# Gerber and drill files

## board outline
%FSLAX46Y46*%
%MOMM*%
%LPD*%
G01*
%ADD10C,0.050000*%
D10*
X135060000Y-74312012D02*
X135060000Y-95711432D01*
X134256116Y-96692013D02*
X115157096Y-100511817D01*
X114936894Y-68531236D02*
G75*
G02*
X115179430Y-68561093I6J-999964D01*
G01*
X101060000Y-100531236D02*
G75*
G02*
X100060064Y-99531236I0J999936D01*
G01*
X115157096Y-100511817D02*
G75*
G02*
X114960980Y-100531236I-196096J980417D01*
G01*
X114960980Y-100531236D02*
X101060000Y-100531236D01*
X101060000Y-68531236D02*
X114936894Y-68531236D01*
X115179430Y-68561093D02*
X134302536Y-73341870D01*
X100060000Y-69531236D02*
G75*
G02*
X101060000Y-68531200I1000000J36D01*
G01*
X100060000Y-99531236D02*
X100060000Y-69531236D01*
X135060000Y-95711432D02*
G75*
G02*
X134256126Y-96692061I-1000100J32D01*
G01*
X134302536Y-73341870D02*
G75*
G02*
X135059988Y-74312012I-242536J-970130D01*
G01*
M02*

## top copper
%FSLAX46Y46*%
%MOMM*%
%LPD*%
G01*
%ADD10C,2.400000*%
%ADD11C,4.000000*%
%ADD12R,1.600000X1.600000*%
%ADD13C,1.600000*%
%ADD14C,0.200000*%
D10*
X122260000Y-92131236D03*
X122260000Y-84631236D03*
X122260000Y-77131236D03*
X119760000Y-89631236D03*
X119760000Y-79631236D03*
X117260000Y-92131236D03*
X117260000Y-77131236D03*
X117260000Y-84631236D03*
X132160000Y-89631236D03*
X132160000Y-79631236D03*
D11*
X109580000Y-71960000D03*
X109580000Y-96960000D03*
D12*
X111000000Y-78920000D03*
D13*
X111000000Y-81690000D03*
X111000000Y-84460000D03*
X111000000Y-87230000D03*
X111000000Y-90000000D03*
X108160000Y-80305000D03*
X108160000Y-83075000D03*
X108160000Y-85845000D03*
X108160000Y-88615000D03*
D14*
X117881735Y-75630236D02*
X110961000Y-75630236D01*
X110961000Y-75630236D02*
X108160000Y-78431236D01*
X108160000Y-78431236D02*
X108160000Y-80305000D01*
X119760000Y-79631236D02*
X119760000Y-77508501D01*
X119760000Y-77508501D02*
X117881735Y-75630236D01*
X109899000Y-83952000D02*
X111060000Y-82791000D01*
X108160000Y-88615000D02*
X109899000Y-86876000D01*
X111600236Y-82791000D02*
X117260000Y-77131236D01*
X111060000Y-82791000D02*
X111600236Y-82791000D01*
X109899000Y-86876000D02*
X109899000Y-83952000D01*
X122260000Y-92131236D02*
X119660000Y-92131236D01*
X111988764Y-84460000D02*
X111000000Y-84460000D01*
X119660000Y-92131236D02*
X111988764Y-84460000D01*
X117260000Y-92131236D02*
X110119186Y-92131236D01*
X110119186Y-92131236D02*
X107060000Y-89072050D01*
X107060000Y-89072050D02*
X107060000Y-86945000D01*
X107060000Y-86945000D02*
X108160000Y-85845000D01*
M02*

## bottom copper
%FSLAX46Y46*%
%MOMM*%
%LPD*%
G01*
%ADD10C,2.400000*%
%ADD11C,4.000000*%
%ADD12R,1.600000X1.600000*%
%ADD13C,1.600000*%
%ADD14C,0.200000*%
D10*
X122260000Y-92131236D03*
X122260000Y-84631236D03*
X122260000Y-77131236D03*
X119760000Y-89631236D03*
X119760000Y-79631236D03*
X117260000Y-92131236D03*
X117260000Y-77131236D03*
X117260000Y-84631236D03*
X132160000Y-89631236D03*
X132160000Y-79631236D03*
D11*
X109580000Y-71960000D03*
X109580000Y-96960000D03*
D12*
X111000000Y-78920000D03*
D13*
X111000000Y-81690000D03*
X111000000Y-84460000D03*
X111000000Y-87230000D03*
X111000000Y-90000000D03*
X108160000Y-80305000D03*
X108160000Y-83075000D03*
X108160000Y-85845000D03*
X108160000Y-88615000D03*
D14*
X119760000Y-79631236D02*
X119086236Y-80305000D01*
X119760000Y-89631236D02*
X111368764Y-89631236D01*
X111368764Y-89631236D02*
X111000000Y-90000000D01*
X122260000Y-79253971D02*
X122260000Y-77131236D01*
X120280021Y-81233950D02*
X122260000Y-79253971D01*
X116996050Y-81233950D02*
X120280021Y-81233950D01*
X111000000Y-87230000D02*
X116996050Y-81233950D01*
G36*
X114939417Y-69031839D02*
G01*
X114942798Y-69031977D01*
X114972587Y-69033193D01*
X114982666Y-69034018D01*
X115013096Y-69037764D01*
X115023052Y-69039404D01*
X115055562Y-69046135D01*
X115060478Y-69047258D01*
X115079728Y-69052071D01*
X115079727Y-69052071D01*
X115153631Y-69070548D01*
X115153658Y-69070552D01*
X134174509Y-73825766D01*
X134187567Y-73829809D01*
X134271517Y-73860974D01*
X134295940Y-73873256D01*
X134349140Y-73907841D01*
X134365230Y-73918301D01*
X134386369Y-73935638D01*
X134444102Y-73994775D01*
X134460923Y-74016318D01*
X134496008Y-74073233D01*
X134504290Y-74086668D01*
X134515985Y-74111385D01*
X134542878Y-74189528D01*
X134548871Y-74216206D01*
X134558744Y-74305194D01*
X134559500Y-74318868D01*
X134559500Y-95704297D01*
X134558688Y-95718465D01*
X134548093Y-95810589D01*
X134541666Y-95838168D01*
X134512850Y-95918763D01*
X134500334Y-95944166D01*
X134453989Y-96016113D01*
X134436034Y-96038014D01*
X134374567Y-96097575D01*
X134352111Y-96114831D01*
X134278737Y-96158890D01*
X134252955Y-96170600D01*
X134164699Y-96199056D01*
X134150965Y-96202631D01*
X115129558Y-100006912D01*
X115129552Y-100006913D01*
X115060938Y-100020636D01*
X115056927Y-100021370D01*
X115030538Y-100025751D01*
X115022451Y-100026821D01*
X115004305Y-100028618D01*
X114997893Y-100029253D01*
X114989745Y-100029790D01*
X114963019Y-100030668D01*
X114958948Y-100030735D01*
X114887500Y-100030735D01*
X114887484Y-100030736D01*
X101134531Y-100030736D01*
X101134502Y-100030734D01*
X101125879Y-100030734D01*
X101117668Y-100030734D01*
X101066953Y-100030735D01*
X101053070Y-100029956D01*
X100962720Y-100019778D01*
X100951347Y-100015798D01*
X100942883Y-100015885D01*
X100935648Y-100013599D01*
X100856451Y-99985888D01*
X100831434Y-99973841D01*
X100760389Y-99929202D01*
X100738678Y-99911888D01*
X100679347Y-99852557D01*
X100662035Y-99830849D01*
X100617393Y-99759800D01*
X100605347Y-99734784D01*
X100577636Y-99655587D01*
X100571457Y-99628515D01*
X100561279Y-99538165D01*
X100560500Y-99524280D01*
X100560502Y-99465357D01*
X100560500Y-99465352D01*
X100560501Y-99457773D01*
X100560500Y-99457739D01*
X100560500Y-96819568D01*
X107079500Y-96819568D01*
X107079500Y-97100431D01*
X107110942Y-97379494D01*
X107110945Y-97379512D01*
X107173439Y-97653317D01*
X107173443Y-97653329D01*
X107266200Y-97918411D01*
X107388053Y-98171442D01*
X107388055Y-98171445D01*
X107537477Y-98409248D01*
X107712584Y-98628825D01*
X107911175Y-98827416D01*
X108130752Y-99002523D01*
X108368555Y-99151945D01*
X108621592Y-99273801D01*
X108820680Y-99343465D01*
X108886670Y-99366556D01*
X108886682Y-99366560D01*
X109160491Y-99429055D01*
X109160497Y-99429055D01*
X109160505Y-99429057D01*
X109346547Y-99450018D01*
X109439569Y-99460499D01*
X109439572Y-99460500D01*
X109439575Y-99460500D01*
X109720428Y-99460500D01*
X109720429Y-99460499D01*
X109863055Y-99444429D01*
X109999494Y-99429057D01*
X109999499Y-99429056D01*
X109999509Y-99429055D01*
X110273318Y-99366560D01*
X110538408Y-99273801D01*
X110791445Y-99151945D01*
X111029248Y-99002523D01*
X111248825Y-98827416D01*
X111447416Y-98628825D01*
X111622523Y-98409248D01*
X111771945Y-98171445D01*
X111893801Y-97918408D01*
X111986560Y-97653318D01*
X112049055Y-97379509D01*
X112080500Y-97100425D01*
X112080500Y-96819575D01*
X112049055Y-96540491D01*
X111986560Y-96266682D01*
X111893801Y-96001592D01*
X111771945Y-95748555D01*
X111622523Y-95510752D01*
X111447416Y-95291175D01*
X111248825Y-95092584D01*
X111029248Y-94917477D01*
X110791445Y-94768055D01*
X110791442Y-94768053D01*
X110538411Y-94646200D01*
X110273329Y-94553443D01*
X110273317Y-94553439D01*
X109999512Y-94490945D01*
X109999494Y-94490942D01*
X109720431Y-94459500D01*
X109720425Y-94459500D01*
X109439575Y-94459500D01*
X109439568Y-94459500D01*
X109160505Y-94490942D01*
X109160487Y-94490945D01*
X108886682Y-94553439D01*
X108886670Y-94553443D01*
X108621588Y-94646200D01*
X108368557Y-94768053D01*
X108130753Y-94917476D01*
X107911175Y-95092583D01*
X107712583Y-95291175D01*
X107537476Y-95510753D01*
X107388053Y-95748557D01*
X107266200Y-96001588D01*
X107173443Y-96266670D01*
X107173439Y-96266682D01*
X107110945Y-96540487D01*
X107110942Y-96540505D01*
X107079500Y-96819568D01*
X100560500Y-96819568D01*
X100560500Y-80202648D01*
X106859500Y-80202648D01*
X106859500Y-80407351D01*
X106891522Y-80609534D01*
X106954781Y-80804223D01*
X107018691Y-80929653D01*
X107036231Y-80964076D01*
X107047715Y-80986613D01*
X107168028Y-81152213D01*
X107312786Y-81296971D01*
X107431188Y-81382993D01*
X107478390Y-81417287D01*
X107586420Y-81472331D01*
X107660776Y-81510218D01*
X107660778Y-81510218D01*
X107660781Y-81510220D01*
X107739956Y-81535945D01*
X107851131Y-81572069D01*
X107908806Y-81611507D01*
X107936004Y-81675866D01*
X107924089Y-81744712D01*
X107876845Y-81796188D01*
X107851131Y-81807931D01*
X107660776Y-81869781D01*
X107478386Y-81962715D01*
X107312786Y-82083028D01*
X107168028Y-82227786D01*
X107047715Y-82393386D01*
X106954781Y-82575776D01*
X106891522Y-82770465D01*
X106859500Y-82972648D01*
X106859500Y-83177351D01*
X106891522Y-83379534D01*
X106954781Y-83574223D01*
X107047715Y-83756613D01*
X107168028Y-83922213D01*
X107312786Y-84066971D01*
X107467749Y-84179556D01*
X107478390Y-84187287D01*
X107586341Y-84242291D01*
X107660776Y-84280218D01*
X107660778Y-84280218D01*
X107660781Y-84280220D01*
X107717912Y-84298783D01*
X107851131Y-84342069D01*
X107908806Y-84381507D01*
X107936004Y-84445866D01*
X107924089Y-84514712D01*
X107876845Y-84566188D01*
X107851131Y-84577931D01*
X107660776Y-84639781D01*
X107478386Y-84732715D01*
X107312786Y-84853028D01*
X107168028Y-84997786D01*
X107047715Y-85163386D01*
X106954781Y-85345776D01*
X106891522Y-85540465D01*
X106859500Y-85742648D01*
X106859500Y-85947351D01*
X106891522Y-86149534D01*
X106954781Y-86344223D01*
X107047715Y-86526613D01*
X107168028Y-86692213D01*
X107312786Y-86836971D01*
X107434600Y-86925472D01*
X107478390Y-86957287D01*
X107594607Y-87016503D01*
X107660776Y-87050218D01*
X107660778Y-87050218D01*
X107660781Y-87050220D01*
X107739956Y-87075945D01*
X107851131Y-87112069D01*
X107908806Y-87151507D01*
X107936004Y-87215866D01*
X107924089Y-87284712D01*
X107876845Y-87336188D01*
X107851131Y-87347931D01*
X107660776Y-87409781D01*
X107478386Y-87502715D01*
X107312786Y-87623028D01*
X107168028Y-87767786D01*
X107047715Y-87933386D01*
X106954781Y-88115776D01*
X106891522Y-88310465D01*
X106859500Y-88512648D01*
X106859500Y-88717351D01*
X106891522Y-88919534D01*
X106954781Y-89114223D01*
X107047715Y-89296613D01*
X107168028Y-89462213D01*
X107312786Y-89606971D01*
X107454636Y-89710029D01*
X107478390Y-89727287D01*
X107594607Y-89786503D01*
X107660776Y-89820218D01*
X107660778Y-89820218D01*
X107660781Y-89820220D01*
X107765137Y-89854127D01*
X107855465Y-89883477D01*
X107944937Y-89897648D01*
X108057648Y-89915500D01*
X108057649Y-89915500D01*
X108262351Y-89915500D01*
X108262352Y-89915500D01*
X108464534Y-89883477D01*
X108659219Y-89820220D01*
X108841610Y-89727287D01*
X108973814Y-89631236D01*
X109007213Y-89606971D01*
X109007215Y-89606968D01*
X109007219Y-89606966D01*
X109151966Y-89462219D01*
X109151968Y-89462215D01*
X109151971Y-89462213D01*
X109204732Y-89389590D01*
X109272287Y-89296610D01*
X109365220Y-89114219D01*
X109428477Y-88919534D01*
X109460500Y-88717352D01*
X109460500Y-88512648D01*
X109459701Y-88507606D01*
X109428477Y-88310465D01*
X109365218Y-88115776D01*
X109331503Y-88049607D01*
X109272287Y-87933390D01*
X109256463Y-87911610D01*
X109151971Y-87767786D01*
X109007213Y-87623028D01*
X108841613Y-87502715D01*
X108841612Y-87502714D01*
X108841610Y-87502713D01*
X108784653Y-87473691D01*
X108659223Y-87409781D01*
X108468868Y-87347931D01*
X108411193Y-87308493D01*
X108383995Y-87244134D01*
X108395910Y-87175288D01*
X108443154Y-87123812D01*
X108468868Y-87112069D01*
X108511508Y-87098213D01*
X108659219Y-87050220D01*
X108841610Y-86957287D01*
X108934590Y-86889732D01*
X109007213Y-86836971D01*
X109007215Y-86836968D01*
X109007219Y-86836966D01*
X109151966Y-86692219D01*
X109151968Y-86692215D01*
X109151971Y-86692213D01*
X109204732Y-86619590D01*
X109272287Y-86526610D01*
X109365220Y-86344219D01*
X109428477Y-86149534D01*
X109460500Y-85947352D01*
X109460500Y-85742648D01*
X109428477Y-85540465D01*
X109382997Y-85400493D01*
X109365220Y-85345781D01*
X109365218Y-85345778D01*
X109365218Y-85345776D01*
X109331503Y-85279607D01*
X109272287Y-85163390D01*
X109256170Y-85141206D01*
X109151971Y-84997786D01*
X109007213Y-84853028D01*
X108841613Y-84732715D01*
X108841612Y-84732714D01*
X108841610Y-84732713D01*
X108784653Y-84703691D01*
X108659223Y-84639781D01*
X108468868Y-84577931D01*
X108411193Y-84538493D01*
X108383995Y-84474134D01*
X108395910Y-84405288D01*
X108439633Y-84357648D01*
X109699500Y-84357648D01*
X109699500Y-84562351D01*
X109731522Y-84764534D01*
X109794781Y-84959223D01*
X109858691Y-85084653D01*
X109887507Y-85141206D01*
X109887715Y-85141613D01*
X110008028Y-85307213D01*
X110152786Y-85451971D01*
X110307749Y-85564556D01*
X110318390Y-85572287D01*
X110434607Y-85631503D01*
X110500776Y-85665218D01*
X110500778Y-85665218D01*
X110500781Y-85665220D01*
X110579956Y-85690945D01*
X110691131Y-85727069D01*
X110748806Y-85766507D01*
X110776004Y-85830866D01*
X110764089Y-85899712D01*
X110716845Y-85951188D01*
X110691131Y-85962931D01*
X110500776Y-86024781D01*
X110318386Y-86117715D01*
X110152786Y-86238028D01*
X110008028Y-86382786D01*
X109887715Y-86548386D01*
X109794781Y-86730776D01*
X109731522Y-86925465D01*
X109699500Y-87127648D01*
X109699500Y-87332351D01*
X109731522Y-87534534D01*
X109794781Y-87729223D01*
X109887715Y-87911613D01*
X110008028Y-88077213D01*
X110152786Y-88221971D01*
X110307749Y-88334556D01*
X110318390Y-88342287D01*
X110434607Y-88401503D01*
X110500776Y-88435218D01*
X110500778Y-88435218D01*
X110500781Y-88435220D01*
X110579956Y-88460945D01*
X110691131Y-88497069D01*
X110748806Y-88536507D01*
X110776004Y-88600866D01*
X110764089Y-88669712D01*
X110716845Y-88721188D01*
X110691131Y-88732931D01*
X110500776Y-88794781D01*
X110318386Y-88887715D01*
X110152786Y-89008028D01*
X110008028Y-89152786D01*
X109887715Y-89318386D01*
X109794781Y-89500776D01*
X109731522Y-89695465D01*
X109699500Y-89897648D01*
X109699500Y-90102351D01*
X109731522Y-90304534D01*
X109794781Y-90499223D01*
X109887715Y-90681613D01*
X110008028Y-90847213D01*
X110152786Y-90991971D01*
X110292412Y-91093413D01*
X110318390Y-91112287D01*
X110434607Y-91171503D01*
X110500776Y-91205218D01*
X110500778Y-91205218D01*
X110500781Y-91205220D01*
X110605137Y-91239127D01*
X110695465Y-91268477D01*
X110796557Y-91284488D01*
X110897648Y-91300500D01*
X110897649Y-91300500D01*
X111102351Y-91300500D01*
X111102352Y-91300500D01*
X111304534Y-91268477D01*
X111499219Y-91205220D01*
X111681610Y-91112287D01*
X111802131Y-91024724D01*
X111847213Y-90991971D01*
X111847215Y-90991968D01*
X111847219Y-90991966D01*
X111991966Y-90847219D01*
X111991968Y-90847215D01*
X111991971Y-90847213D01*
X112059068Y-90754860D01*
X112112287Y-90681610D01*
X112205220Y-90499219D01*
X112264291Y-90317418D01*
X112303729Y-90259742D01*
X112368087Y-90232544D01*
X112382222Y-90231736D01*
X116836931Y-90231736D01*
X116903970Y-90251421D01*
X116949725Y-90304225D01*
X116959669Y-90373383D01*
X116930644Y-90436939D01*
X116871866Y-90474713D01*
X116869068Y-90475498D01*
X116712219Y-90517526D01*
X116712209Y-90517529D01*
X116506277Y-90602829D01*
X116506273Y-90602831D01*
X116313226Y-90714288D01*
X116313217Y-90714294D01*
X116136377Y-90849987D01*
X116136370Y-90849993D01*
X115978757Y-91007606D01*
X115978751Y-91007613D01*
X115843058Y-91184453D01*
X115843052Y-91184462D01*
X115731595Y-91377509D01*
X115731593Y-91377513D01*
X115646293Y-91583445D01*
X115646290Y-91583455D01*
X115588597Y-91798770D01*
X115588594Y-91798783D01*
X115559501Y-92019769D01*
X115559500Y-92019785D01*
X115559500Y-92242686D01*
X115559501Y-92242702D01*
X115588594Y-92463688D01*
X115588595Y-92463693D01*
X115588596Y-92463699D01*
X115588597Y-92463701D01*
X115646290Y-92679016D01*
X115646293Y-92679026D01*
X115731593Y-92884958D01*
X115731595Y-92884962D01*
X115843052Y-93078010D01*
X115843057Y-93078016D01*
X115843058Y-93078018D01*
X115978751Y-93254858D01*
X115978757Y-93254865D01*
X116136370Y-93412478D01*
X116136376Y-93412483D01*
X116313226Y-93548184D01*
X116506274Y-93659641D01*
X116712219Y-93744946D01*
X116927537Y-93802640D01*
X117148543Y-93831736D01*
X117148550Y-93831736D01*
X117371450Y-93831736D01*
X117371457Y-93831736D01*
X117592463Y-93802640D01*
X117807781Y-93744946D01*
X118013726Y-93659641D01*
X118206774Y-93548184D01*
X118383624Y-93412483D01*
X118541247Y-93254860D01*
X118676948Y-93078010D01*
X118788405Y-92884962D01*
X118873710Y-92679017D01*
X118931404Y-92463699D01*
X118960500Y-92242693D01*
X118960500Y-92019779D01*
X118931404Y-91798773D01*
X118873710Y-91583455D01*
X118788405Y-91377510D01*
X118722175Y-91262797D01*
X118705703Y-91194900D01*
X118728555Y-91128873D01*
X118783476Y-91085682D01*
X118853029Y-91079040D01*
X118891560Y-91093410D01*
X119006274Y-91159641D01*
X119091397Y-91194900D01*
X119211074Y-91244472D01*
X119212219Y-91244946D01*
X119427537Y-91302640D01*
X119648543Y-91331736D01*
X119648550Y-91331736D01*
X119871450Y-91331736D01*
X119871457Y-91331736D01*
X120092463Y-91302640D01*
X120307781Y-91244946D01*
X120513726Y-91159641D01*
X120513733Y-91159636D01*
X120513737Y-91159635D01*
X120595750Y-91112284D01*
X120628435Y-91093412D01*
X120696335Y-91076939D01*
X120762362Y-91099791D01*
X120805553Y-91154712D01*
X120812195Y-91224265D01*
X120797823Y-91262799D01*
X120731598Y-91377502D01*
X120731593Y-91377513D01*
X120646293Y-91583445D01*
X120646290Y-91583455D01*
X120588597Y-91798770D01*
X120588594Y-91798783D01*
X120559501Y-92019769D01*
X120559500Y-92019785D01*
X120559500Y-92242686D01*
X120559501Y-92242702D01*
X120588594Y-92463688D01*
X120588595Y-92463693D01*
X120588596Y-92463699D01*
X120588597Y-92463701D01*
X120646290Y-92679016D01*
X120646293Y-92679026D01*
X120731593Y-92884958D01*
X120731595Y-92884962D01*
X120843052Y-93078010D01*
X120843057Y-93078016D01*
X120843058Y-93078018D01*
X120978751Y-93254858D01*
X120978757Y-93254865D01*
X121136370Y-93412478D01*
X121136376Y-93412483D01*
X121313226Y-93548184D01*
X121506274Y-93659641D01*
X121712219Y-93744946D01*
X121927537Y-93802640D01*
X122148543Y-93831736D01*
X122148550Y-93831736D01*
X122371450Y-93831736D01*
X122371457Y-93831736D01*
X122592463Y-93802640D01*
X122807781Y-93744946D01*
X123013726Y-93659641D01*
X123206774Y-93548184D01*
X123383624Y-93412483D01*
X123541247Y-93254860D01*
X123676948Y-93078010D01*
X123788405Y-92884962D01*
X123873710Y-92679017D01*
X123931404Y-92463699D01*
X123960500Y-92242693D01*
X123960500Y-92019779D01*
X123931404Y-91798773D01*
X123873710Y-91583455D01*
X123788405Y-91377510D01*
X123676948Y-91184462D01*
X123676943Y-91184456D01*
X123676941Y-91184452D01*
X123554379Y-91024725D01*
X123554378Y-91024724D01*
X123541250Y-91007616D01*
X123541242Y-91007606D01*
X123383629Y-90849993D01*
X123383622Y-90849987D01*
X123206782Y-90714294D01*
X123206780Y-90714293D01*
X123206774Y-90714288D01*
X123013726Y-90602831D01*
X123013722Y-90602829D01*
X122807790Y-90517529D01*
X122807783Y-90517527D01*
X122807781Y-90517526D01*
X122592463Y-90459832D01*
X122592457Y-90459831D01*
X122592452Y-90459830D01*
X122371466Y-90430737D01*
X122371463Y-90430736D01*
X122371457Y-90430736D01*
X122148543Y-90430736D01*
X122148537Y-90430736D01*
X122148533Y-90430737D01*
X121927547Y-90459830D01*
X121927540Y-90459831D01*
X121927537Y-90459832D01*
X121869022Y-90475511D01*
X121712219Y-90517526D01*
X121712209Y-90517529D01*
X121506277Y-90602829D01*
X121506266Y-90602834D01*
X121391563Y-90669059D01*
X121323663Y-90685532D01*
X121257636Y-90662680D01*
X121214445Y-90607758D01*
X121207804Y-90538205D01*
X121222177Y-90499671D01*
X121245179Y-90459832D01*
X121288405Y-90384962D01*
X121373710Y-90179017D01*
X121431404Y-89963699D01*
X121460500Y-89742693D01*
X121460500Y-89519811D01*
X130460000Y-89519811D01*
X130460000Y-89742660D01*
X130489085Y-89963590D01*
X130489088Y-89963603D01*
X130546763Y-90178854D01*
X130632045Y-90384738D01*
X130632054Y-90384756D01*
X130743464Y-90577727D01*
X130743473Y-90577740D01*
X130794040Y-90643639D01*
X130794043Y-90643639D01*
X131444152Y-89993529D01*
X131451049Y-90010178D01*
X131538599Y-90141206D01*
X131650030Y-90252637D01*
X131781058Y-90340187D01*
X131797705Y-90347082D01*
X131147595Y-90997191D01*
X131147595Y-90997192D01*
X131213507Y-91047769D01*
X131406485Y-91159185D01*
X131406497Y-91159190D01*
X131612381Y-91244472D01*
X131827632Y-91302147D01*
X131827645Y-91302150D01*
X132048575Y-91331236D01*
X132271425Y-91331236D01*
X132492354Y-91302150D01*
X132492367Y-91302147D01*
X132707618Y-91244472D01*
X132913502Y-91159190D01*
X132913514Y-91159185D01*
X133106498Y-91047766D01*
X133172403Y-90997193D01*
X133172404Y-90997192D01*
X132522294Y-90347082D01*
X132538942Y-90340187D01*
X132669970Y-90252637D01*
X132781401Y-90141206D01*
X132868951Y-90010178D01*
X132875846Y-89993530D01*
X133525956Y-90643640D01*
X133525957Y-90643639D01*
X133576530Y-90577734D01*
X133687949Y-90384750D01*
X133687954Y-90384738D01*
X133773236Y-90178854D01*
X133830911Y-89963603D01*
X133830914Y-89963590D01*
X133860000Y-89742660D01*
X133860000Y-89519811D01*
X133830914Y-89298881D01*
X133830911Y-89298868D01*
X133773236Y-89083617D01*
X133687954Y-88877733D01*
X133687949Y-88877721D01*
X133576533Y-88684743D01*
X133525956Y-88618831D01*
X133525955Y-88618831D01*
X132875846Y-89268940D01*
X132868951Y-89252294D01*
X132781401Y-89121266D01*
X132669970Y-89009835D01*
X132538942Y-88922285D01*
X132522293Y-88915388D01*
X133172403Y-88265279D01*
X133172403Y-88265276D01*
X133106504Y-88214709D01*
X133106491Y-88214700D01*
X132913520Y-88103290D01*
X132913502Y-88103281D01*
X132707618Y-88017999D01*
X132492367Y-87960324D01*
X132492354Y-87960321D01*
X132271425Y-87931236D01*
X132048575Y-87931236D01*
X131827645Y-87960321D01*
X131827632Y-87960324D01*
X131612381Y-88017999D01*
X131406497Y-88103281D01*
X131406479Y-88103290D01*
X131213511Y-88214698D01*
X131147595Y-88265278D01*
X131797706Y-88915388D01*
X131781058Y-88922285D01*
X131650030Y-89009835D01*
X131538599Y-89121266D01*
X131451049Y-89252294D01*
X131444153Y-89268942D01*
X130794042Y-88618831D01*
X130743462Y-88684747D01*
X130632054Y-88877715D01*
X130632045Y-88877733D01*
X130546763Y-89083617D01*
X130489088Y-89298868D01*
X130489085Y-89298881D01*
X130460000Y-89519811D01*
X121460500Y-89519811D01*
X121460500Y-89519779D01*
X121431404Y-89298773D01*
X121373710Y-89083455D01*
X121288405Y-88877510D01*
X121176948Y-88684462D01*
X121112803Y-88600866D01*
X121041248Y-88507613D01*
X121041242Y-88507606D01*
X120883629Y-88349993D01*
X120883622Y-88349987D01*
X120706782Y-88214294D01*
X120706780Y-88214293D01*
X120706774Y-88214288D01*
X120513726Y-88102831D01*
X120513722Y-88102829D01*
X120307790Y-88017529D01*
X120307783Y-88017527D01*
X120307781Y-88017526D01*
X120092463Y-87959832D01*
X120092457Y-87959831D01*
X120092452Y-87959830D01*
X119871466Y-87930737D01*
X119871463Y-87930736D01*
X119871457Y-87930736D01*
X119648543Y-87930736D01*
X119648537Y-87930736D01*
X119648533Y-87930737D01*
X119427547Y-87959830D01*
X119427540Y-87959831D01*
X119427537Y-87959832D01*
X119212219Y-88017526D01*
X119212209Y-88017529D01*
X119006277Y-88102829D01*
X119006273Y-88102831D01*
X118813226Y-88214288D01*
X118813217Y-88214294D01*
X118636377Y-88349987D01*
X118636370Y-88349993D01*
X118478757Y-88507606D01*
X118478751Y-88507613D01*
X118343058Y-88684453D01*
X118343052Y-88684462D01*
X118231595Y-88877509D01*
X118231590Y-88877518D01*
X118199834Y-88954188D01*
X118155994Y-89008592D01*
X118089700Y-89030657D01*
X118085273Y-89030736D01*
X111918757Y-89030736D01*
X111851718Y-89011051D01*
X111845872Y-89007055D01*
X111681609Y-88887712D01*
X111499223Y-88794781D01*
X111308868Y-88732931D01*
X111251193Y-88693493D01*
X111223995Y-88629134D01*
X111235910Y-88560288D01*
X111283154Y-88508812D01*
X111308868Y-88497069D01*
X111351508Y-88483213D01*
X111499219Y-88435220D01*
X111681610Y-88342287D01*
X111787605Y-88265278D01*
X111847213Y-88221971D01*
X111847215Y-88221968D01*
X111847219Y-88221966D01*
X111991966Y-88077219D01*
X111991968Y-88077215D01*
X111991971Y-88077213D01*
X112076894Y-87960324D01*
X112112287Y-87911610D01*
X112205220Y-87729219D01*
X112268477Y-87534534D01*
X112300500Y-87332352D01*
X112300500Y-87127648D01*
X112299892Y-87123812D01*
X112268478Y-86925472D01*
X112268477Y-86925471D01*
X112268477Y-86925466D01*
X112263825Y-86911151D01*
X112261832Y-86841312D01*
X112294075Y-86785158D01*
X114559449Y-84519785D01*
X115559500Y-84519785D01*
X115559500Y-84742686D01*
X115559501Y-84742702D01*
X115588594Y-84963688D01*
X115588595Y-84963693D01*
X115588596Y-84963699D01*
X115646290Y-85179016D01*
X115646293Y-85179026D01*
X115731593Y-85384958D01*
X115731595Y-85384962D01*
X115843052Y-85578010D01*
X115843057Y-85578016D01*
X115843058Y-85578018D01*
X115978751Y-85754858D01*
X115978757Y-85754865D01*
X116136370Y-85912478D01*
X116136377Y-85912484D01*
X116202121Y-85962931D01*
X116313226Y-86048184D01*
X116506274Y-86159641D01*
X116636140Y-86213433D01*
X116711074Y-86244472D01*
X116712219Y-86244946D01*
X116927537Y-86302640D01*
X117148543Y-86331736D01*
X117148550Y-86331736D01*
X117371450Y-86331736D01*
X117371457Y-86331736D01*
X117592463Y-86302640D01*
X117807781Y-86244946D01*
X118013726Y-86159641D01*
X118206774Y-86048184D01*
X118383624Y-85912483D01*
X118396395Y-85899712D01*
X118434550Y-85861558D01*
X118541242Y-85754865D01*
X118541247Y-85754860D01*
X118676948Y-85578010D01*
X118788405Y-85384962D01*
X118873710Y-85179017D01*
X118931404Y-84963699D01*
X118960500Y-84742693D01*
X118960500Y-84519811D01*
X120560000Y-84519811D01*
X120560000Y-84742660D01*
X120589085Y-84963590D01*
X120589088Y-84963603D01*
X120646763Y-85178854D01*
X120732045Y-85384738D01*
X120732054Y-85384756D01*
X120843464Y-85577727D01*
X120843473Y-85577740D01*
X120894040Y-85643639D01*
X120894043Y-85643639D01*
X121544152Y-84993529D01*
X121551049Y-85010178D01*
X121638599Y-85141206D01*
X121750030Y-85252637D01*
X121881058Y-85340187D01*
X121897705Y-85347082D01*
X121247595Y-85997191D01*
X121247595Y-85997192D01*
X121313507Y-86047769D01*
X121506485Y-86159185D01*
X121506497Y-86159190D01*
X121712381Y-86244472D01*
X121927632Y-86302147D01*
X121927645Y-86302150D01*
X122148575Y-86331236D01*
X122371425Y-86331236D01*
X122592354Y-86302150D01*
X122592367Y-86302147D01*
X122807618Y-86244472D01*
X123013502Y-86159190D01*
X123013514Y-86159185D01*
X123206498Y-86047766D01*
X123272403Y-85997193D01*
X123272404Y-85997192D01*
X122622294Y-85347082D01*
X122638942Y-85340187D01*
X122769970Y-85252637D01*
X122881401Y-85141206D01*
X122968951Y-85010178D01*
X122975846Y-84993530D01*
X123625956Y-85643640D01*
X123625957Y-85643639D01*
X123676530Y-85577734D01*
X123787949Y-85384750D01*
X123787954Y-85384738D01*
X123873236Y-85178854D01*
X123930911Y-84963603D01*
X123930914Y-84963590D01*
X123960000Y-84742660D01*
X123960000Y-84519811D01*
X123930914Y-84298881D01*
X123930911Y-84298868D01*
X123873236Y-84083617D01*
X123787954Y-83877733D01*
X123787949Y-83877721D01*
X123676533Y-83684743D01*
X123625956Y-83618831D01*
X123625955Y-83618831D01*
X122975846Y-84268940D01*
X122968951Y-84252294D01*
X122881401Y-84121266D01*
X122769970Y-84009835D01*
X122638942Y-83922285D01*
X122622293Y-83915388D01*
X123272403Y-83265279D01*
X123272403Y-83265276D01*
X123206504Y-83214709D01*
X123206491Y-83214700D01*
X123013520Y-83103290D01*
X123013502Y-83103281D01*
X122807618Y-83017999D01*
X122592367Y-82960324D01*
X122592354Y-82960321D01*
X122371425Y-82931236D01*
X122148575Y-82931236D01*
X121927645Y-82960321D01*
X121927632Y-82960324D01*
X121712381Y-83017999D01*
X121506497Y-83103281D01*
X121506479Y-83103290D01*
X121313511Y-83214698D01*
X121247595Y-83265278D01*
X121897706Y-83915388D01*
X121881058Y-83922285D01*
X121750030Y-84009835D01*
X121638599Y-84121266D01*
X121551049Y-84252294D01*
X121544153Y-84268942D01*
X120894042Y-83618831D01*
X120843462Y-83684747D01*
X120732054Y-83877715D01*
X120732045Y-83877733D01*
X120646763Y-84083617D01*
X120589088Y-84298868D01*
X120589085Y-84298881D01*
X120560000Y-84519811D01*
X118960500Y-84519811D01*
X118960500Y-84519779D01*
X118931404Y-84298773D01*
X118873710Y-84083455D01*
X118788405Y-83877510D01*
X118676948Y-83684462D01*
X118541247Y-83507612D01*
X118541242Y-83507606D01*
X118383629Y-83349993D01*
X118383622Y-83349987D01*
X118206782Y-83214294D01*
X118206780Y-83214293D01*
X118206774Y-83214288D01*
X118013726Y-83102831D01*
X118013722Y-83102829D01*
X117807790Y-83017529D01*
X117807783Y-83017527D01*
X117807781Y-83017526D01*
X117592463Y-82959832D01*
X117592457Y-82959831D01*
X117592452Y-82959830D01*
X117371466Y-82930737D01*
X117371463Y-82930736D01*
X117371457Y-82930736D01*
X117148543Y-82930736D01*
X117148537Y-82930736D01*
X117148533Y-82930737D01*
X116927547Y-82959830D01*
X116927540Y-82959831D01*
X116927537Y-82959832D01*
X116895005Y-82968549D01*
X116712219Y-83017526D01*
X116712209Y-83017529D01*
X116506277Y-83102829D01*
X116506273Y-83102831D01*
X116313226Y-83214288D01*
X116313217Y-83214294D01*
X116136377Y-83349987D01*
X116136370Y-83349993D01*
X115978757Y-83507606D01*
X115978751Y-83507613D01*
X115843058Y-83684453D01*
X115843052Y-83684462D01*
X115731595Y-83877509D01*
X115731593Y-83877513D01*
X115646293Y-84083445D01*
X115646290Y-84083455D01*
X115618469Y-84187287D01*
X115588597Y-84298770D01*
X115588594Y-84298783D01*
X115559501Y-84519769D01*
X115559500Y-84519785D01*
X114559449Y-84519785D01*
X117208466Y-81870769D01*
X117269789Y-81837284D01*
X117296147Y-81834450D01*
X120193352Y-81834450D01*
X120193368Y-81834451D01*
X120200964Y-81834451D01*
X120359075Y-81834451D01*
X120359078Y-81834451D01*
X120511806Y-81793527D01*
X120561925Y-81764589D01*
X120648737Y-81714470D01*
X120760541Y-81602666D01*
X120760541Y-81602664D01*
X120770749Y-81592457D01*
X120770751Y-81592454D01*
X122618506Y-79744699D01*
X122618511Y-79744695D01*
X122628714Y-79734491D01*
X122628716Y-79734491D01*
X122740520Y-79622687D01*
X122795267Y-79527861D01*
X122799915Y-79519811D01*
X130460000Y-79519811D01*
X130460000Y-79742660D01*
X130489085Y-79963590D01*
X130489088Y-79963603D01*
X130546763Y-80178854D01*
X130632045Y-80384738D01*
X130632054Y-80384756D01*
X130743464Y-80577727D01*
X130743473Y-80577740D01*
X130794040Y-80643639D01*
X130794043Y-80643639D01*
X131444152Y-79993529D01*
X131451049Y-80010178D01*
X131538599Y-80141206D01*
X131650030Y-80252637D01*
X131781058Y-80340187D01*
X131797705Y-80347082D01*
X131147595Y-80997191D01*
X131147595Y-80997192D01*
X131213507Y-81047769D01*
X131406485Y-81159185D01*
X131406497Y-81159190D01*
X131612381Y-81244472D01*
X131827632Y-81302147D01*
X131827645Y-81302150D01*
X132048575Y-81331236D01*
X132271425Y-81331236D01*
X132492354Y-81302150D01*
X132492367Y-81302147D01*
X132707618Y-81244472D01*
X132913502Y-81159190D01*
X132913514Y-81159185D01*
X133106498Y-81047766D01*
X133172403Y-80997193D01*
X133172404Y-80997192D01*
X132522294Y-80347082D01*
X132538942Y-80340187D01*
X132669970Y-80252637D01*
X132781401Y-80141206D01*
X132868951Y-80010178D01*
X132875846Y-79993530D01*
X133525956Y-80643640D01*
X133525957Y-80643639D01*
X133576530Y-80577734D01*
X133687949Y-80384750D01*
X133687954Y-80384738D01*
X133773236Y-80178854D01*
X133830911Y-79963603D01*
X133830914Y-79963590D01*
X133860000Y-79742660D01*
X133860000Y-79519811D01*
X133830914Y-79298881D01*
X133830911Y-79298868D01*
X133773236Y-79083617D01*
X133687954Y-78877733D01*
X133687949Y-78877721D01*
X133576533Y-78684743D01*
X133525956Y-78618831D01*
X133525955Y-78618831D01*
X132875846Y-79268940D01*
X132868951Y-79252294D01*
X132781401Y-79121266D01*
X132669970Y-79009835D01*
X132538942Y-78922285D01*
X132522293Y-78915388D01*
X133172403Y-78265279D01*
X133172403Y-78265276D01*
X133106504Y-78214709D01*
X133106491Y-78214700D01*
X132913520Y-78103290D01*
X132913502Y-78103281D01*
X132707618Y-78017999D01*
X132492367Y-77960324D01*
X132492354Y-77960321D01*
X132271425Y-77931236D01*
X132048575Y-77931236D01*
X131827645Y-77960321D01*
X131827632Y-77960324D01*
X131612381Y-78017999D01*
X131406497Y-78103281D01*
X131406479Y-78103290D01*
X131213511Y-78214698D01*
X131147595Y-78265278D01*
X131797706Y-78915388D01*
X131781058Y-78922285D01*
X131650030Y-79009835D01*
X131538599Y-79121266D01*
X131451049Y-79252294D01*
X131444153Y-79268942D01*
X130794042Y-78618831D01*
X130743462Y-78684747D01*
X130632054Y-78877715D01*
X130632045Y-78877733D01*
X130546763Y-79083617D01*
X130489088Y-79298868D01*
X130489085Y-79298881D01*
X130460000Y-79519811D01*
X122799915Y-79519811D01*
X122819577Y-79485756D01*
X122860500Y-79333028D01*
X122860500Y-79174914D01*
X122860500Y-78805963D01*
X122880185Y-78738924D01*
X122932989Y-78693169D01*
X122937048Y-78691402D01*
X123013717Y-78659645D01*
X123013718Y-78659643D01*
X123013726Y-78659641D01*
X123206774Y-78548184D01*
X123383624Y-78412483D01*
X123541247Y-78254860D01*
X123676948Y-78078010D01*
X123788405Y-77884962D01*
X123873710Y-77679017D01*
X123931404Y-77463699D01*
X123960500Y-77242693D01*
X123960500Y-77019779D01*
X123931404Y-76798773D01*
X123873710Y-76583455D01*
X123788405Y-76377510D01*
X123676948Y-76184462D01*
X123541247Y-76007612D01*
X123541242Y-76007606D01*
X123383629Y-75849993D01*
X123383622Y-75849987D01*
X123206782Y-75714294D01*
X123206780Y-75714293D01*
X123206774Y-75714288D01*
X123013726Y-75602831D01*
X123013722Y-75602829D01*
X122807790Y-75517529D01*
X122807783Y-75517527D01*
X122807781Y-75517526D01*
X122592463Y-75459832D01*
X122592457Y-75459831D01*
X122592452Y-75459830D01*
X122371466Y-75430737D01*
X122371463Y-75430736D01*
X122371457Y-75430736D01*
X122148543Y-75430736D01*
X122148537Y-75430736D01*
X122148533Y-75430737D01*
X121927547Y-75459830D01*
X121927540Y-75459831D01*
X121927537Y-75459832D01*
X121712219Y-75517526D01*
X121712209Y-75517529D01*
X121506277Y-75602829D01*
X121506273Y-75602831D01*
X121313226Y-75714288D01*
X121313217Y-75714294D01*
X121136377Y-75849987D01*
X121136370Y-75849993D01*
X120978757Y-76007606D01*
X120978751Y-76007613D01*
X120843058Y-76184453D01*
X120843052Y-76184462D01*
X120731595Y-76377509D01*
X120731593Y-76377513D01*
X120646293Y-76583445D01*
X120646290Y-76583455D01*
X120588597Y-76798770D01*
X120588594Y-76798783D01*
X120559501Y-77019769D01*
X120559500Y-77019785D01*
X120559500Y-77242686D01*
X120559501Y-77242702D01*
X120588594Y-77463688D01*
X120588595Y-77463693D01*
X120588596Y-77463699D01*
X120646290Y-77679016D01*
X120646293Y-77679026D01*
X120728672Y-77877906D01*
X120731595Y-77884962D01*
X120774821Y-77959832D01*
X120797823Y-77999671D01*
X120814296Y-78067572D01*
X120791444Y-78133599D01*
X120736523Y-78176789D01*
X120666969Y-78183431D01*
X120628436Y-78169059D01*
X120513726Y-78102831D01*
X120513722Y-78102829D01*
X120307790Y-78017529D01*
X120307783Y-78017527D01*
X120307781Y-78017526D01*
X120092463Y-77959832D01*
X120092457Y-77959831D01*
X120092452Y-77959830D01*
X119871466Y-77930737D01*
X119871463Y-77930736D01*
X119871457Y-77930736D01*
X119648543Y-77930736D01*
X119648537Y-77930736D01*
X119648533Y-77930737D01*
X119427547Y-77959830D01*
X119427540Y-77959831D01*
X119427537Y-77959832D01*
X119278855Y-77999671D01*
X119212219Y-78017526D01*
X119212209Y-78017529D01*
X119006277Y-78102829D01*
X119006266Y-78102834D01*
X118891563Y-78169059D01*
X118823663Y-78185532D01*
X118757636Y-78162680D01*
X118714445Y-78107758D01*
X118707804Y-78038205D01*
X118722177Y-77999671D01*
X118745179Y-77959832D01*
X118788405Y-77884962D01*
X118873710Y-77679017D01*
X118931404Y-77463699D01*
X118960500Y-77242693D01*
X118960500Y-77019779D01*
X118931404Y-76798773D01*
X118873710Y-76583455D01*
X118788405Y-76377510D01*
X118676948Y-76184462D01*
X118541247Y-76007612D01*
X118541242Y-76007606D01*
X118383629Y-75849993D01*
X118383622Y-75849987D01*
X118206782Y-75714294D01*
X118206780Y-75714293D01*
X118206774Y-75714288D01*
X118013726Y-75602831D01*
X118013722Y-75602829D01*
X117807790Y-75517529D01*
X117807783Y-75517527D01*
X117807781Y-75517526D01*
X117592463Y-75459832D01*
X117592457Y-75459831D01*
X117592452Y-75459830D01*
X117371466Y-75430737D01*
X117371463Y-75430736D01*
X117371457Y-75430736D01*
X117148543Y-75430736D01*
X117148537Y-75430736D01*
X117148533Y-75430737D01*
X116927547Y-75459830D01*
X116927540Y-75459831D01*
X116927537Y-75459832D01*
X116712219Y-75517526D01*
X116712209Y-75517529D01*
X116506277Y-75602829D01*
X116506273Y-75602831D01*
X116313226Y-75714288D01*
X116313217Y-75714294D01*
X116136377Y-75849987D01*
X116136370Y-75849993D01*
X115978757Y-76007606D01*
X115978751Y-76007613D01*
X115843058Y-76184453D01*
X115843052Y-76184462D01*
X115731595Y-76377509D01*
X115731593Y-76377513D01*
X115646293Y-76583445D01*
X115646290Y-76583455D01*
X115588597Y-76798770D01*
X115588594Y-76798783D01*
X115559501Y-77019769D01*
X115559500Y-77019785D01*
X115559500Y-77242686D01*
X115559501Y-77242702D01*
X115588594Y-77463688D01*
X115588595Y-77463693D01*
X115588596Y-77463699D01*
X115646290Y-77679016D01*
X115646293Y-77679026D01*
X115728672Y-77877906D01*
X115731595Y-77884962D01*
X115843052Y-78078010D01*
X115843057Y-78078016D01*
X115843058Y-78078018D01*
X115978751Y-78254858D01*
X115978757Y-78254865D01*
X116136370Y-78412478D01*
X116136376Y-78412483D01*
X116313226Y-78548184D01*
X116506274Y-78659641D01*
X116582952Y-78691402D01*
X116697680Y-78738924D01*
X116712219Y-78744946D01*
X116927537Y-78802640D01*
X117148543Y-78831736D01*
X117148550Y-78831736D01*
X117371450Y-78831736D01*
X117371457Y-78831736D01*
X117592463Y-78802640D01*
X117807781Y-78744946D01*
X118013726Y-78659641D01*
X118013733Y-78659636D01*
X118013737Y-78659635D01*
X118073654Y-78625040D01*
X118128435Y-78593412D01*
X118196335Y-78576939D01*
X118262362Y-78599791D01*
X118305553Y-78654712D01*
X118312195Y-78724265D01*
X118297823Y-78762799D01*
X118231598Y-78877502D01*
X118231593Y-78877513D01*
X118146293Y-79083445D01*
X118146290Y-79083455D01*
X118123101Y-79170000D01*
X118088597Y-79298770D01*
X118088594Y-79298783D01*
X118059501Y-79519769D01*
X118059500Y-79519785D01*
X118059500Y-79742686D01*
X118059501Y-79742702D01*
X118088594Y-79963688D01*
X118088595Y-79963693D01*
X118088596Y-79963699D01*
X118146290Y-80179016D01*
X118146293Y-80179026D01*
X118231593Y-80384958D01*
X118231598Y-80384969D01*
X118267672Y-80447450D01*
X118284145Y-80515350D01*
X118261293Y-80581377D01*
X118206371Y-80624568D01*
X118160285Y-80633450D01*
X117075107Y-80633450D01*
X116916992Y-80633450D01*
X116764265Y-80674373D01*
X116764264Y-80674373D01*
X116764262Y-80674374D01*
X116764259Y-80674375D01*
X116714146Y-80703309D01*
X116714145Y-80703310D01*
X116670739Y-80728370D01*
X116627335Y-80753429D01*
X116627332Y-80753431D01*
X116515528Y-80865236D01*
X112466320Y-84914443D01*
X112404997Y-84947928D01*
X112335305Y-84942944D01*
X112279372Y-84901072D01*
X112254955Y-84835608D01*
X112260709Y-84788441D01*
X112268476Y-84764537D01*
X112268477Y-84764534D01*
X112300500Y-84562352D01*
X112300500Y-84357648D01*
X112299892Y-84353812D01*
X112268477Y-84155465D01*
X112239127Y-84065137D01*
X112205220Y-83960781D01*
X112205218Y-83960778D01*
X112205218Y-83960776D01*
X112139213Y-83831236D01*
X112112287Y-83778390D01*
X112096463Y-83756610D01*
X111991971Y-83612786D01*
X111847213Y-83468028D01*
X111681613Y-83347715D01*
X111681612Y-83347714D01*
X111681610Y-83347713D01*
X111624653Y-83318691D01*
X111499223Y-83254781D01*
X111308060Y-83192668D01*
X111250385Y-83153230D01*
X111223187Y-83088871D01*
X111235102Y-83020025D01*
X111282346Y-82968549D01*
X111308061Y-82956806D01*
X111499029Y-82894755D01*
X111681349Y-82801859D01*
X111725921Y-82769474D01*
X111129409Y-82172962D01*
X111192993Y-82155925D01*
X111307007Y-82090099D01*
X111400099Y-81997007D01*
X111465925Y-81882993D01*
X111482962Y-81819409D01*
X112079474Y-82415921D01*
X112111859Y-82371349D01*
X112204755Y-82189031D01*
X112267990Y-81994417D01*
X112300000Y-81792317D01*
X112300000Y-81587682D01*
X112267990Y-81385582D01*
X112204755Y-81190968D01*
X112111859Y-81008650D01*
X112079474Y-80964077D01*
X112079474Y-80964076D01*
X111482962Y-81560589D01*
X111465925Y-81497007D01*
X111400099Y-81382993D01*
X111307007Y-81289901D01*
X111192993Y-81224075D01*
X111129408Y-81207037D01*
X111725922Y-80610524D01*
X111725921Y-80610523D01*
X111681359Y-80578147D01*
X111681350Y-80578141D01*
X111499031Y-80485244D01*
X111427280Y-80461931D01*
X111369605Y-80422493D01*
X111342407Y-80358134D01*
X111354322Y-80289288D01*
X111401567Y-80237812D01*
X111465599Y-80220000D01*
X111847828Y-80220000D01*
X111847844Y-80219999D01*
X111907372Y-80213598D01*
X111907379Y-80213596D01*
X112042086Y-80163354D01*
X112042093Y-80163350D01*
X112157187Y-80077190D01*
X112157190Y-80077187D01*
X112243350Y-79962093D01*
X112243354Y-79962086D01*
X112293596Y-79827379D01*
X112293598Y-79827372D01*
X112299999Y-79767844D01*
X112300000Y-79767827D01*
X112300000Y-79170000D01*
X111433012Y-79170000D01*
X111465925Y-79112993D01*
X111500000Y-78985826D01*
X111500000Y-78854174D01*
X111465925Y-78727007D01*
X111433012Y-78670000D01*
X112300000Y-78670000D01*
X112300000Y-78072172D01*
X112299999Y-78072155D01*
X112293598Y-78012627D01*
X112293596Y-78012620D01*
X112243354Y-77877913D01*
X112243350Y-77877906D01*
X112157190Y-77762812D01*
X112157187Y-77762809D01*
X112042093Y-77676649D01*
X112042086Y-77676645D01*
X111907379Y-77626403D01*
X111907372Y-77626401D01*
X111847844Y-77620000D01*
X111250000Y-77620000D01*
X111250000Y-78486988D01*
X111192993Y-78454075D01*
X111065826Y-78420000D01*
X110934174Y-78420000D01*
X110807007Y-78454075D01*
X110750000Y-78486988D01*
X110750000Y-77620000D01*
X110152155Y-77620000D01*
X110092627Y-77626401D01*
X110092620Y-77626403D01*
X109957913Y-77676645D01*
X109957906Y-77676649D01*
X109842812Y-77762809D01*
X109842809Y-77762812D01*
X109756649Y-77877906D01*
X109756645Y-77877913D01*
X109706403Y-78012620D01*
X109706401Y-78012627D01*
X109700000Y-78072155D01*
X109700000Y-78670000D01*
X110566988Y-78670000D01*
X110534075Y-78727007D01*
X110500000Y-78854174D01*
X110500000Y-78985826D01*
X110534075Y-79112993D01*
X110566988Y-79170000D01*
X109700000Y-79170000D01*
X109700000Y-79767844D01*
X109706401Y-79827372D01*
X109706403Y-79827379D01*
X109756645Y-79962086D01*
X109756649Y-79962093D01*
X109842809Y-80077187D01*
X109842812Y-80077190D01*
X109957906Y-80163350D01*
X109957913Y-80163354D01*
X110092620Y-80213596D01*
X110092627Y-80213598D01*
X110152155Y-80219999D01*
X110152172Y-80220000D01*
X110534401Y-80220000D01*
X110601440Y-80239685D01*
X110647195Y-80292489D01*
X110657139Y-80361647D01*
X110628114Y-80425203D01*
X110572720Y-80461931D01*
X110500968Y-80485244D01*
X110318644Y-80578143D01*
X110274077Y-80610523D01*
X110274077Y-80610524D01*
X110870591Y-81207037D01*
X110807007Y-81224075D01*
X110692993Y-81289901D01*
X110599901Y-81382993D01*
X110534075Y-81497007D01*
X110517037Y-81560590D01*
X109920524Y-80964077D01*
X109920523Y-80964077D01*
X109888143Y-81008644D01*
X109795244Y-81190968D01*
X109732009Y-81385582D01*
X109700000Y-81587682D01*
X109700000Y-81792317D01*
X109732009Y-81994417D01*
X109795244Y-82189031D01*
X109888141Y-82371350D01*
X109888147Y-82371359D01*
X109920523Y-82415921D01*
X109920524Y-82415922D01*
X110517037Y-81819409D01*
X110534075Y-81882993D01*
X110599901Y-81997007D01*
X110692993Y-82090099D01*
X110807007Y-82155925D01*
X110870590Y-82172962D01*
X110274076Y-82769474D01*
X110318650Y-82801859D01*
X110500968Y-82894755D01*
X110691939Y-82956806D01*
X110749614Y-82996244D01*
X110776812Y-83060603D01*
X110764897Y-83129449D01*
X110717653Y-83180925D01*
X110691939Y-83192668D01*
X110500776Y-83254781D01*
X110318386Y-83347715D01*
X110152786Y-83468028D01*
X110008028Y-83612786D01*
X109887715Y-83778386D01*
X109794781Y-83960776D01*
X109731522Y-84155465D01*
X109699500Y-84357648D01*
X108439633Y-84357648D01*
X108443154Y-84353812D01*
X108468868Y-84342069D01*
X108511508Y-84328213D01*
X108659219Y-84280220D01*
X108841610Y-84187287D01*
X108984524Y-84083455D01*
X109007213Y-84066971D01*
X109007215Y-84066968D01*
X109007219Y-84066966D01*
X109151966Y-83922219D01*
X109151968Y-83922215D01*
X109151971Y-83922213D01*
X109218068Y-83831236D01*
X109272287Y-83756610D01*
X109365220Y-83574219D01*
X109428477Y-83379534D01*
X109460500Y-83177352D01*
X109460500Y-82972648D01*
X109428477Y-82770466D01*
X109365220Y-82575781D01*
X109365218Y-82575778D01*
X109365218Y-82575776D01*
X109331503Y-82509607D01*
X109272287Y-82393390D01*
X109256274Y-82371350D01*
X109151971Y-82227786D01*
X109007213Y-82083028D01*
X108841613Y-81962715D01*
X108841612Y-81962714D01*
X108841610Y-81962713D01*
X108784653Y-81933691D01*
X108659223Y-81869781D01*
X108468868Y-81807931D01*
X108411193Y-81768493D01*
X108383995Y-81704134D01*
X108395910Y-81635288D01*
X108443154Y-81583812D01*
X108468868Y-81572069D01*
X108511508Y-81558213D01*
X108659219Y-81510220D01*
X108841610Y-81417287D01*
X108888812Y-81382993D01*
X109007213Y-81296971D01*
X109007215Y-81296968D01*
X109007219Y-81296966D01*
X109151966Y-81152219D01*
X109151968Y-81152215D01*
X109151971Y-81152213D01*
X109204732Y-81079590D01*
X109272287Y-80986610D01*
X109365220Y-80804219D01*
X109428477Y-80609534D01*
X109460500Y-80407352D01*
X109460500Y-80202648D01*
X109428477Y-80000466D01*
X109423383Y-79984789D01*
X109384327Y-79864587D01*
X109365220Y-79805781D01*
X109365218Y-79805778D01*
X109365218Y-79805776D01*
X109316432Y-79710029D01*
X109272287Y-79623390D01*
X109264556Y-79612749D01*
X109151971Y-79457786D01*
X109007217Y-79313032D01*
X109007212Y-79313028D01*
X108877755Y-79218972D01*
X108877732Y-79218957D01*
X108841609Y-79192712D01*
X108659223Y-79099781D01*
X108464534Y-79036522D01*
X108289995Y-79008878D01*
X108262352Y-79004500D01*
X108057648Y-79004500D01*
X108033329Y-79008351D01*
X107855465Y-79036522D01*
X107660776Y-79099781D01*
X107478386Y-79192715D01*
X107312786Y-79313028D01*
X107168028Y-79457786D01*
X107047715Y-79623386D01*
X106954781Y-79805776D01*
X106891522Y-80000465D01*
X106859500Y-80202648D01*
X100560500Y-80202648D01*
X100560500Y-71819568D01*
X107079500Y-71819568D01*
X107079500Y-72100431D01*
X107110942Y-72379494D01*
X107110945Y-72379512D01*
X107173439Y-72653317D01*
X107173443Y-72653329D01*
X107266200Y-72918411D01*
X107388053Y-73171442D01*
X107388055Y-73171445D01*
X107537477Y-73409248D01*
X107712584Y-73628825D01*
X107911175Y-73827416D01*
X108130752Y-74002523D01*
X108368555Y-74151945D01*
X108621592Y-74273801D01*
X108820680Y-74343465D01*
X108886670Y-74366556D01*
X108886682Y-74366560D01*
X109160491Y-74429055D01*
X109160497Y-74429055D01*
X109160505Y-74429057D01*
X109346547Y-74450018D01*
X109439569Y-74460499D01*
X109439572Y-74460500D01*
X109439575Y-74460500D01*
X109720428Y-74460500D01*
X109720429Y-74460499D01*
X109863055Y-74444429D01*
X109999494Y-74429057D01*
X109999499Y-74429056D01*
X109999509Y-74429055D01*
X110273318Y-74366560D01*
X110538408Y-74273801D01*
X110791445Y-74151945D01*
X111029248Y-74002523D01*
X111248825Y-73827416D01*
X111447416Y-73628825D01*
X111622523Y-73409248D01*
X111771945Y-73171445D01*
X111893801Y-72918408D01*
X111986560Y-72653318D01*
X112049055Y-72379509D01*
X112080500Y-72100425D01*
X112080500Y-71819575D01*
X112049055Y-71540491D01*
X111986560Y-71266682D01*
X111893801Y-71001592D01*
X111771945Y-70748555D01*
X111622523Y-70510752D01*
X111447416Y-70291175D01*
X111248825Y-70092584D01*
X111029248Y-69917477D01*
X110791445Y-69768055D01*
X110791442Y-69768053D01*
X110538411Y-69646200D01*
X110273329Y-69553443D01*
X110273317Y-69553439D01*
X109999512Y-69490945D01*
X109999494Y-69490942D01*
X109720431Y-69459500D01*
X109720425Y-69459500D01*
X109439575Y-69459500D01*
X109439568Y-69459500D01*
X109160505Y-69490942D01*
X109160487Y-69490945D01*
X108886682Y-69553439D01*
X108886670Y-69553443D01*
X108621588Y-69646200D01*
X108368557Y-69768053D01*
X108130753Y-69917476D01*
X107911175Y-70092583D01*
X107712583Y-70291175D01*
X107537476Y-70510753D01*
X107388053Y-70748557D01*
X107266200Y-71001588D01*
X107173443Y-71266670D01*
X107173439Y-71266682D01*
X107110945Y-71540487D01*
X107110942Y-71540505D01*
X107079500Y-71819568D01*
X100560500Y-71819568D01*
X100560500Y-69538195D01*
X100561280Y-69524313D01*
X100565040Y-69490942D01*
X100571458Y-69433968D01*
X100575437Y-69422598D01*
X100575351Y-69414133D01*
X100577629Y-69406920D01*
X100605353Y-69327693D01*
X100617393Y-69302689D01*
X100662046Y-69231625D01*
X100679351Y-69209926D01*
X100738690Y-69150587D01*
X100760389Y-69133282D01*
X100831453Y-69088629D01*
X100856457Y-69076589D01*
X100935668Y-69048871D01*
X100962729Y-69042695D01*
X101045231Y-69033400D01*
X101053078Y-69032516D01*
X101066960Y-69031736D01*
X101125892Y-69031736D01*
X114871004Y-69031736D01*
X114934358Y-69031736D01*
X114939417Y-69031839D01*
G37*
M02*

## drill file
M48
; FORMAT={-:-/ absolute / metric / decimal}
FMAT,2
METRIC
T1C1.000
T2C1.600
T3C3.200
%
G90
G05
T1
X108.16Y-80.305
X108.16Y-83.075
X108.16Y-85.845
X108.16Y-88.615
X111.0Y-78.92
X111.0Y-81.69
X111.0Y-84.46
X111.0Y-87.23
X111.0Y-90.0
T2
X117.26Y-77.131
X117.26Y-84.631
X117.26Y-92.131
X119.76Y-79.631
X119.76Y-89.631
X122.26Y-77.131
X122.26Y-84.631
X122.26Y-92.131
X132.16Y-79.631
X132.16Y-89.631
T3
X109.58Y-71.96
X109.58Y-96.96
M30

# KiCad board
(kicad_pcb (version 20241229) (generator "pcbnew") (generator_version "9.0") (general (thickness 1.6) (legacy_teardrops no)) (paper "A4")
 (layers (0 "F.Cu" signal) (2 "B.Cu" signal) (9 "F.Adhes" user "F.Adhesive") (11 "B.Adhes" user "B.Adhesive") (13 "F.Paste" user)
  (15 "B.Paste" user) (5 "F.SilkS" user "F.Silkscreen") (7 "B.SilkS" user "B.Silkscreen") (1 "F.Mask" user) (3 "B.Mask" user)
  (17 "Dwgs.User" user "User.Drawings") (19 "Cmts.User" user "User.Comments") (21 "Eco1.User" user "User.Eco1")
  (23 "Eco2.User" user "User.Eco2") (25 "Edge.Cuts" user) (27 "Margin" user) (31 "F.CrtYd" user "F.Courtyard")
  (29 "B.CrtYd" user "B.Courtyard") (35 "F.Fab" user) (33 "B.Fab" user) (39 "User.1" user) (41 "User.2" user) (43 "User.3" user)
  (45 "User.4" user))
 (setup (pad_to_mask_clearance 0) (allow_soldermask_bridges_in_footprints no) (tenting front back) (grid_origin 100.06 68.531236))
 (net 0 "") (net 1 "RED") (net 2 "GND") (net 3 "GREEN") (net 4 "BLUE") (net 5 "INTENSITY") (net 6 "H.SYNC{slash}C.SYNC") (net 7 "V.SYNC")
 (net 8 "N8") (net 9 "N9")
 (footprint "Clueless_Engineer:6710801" (layer "F.Cu") (at 122.26 92.131236 -90)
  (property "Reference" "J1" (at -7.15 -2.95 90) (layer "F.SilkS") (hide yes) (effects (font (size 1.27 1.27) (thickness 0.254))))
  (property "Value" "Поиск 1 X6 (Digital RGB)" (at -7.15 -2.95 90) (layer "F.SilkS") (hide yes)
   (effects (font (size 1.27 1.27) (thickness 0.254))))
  (pad "1" thru_hole circle (at 0 0 270) (size 2.4 2.4) (drill 1.6) (layers "*.Cu" "*.Mask") (remove_unused_layers no) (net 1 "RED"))
  (pad "2" thru_hole circle (at -7.5 0 270) (size 2.4 2.4) (drill 1.6) (layers "*.Cu" "*.Mask") (remove_unused_layers no) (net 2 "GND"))
  (pad "3" thru_hole circle (at -15 0 270) (size 2.4 2.4) (drill 1.6) (layers "*.Cu" "*.Mask") (remove_unused_layers no) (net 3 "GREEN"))
  (pad "4" thru_hole circle (at -2.5 2.5 270) (size 2.4 2.4) (drill 1.6) (layers "*.Cu" "*.Mask") (remove_unused_layers no) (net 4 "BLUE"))
  (pad "5" thru_hole circle (at -12.5 2.5 270) (size 2.4 2.4) (drill 1.6) (layers "*.Cu" "*.Mask") (remove_unused_layers no)
   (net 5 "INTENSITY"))
  (pad "6" thru_hole circle (at 0 5 270) (size 2.4 2.4) (drill 1.6) (layers "*.Cu" "*.Mask") (remove_unused_layers no)
   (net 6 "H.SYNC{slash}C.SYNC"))
  (pad "7" thru_hole circle (at -15 5 270) (size 2.4 2.4) (drill 1.6) (layers "*.Cu" "*.Mask") (remove_unused_layers no) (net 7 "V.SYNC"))
  (pad "8" thru_hole circle (at -7.5 5 270) (size 2.4 2.4) (drill 1.6) (layers "*.Cu" "*.Mask") (remove_unused_layers no) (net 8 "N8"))
  (pad "MH1" thru_hole circle (at -2.5 -9.9 270) (size 2.4 2.4) (drill 1.6) (layers "*.Cu" "*.Mask") (remove_unused_layers no) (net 2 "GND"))
  (pad "MH2" thru_hole circle (at -12.5 -9.9 270) (size 2.4 2.4) (drill 1.6) (layers "*.Cu" "*.Mask") (remove_unused_layers no)
   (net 2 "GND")))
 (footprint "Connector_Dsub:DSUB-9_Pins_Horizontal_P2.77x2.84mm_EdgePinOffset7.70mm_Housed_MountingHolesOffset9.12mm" (layer "F.Cu")
  (at 111 78.92 -90)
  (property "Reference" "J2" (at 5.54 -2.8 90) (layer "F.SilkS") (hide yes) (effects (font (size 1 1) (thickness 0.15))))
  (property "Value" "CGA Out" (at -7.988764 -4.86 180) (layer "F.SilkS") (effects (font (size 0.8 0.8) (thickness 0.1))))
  (pad "0" thru_hole circle (at -6.96 1.42 270) (size 4 4) (drill 3.2) (layers "*.Cu" "*.Mask") (remove_unused_layers no))
  (pad "0" thru_hole circle (at 18.04 1.42 270) (size 4 4) (drill 3.2) (layers "*.Cu" "*.Mask") (remove_unused_layers no))
  (pad "1" thru_hole rect (at 0 0 270) (size 1.6 1.6) (drill 1) (layers "*.Cu" "*.Mask") (remove_unused_layers no) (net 2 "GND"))
  (pad "2" thru_hole circle (at 2.77 0 270) (size 1.6 1.6) (drill 1) (layers "*.Cu" "*.Mask") (remove_unused_layers no) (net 2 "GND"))
  (pad "3" thru_hole circle (at 5.54 0 270) (size 1.6 1.6) (drill 1) (layers "*.Cu" "*.Mask") (remove_unused_layers no) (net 1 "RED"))
  (pad "4" thru_hole circle (at 8.31 0 270) (size 1.6 1.6) (drill 1) (layers "*.Cu" "*.Mask") (remove_unused_layers no) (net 3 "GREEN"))
  (pad "5" thru_hole circle (at 11.08 0 270) (size 1.6 1.6) (drill 1) (layers "*.Cu" "*.Mask") (remove_unused_layers no) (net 4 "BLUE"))
  (pad "6" thru_hole circle (at 1.385 2.84 270) (size 1.6 1.6) (drill 1) (layers "*.Cu" "*.Mask") (remove_unused_layers no)
   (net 5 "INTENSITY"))
  (pad "7" thru_hole circle (at 4.155 2.84 270) (size 1.6 1.6) (drill 1) (layers "*.Cu" "*.Mask") (remove_unused_layers no) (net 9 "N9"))
  (pad "8" thru_hole circle (at 6.925 2.84 270) (size 1.6 1.6) (drill 1) (layers "*.Cu" "*.Mask") (remove_unused_layers no)
   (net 6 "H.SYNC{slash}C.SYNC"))
  (pad "9" thru_hole circle (at 9.695 2.84 270) (size 1.6 1.6) (drill 1) (layers "*.Cu" "*.Mask") (remove_unused_layers no) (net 7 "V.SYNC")))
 (gr_line (start 135.06 74.312012) (end 135.06 95.711432) (stroke (width 0.05) (type default)) (layer "Edge.Cuts"))
 (gr_line (start 134.256116 96.692013) (end 115.157096 100.511817) (stroke (width 0.05) (type default)) (layer "Edge.Cuts"))
 (gr_arc (start 114.936894 68.531236) (mid 115.059077 68.538728) (end 115.17943 68.561093) (stroke (width 0.05) (type default))
  (layer "Edge.Cuts"))
 (gr_arc (start 101.06 100.531236) (mid 100.35288 100.238345) (end 100.06 99.531236) (stroke (width 0.05) (type default))
  (layer "Edge.Cuts"))
 (gr_arc (start 115.157096 100.511817) (mid 115.059518 100.52637) (end 114.96098 100.531236) (stroke (width 0.05) (type default))
  (layer "Edge.Cuts"))
 (gr_line (start 114.96098 100.531236) (end 101.06 100.531236) (stroke (width 0.05) (type default)) (layer "Edge.Cuts"))
 (gr_line (start 101.06 68.531236) (end 114.936894 68.531236) (stroke (width 0.05) (type default)) (layer "Edge.Cuts"))
 (gr_line (start 115.17943 68.561093) (end 134.302536 73.34187) (stroke (width 0.05) (type default)) (layer "Edge.Cuts"))
 (gr_arc (start 100.06 69.531236) (mid 100.352893 68.824129) (end 101.06 68.531236) (stroke (width 0.05) (type default)) (layer "Edge.Cuts"))
 (gr_line (start 100.06 99.531236) (end 100.06 69.531236) (stroke (width 0.05) (type default)) (layer "Edge.Cuts"))
 (gr_arc (start 135.06 95.711432) (mid 134.83333 96.345404) (end 134.256116 96.692013) (stroke (width 0.05) (type default))
  (layer "Edge.Cuts"))
 (gr_arc (start 134.302536 73.34187) (mid 134.848205 73.6966) (end 135.06 74.312012) (stroke (width 0.05) (type default))
  (layer "Edge.Cuts"))
 (segment (start 117.881735 75.630236) (end 110.961 75.630236) (width 0.2) (layer "F.Cu") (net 5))
 (segment (start 110.961 75.630236) (end 108.16 78.431236) (width 0.2) (layer "F.Cu") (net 5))
 (segment (start 108.16 78.431236) (end 108.16 80.305) (width 0.2) (layer "F.Cu") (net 5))
 (segment (start 119.76 79.631236) (end 119.76 77.508501) (width 0.2) (layer "F.Cu") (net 5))
 (segment (start 119.76 77.508501) (end 117.881735 75.630236) (width 0.2) (layer "F.Cu") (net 5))
 (segment (start 119.76 79.631236) (end 119.086236 80.305) (width 0.2) (layer "B.Cu") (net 5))
 (segment (start 109.899 83.952) (end 111.06 82.791) (width 0.2) (layer "F.Cu") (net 7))
 (segment (start 108.16 88.615) (end 109.899 86.876) (width 0.2) (layer "F.Cu") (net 7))
 (segment (start 111.600236 82.791) (end 117.26 77.131236) (width 0.2) (layer "F.Cu") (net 7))
 (segment (start 111.06 82.791) (end 111.600236 82.791) (width 0.2) (layer "F.Cu") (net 7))
 (segment (start 109.899 86.876) (end 109.899 83.952) (width 0.2) (layer "F.Cu") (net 7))
 (segment (start 122.26 92.131236) (end 119.66 92.131236) (width 0.2) (layer "F.Cu") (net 1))
 (segment (start 111.988764 84.46) (end 111 84.46) (width 0.2) (layer "F.Cu") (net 1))
 (segment (start 119.66 92.131236) (end 111.988764 84.46) (width 0.2) (layer "F.Cu") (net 1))
 (segment (start 117.26 92.131236) (end 110.119186 92.131236) (width 0.2) (layer "F.Cu") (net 6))
 (segment (start 110.119186 92.131236) (end 107.06 89.07205) (width 0.2) (layer "F.Cu") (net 6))
 (segment (start 107.06 89.07205) (end 107.06 86.945) (width 0.2) (layer "F.Cu") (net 6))
 (segment (start 107.06 86.945) (end 108.16 85.845) (width 0.2) (layer "F.Cu") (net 6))
 (segment (start 119.76 89.631236) (end 111.368764 89.631236) (width 0.2) (layer "B.Cu") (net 4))
 (segment (start 111.368764 89.631236) (end 111 90) (width 0.2) (layer "B.Cu") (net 4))
 (segment (start 122.26 79.253971) (end 122.26 77.131236) (width 0.2) (layer "B.Cu") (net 3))
 (segment (start 120.280021 81.23395) (end 122.26 79.253971) (width 0.2) (layer "B.Cu") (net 3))
 (segment (start 116.99605 81.23395) (end 120.280021 81.23395) (width 0.2) (layer "B.Cu") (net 3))
 (segment (start 111 87.23) (end 116.99605 81.23395) (width 0.2) (layer "B.Cu") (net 3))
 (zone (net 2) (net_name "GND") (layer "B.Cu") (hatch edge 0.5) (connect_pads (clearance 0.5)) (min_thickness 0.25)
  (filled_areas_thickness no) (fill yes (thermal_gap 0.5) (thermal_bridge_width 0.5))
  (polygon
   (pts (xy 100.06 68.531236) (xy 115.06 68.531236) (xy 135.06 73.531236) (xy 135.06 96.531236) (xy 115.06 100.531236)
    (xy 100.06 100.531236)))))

